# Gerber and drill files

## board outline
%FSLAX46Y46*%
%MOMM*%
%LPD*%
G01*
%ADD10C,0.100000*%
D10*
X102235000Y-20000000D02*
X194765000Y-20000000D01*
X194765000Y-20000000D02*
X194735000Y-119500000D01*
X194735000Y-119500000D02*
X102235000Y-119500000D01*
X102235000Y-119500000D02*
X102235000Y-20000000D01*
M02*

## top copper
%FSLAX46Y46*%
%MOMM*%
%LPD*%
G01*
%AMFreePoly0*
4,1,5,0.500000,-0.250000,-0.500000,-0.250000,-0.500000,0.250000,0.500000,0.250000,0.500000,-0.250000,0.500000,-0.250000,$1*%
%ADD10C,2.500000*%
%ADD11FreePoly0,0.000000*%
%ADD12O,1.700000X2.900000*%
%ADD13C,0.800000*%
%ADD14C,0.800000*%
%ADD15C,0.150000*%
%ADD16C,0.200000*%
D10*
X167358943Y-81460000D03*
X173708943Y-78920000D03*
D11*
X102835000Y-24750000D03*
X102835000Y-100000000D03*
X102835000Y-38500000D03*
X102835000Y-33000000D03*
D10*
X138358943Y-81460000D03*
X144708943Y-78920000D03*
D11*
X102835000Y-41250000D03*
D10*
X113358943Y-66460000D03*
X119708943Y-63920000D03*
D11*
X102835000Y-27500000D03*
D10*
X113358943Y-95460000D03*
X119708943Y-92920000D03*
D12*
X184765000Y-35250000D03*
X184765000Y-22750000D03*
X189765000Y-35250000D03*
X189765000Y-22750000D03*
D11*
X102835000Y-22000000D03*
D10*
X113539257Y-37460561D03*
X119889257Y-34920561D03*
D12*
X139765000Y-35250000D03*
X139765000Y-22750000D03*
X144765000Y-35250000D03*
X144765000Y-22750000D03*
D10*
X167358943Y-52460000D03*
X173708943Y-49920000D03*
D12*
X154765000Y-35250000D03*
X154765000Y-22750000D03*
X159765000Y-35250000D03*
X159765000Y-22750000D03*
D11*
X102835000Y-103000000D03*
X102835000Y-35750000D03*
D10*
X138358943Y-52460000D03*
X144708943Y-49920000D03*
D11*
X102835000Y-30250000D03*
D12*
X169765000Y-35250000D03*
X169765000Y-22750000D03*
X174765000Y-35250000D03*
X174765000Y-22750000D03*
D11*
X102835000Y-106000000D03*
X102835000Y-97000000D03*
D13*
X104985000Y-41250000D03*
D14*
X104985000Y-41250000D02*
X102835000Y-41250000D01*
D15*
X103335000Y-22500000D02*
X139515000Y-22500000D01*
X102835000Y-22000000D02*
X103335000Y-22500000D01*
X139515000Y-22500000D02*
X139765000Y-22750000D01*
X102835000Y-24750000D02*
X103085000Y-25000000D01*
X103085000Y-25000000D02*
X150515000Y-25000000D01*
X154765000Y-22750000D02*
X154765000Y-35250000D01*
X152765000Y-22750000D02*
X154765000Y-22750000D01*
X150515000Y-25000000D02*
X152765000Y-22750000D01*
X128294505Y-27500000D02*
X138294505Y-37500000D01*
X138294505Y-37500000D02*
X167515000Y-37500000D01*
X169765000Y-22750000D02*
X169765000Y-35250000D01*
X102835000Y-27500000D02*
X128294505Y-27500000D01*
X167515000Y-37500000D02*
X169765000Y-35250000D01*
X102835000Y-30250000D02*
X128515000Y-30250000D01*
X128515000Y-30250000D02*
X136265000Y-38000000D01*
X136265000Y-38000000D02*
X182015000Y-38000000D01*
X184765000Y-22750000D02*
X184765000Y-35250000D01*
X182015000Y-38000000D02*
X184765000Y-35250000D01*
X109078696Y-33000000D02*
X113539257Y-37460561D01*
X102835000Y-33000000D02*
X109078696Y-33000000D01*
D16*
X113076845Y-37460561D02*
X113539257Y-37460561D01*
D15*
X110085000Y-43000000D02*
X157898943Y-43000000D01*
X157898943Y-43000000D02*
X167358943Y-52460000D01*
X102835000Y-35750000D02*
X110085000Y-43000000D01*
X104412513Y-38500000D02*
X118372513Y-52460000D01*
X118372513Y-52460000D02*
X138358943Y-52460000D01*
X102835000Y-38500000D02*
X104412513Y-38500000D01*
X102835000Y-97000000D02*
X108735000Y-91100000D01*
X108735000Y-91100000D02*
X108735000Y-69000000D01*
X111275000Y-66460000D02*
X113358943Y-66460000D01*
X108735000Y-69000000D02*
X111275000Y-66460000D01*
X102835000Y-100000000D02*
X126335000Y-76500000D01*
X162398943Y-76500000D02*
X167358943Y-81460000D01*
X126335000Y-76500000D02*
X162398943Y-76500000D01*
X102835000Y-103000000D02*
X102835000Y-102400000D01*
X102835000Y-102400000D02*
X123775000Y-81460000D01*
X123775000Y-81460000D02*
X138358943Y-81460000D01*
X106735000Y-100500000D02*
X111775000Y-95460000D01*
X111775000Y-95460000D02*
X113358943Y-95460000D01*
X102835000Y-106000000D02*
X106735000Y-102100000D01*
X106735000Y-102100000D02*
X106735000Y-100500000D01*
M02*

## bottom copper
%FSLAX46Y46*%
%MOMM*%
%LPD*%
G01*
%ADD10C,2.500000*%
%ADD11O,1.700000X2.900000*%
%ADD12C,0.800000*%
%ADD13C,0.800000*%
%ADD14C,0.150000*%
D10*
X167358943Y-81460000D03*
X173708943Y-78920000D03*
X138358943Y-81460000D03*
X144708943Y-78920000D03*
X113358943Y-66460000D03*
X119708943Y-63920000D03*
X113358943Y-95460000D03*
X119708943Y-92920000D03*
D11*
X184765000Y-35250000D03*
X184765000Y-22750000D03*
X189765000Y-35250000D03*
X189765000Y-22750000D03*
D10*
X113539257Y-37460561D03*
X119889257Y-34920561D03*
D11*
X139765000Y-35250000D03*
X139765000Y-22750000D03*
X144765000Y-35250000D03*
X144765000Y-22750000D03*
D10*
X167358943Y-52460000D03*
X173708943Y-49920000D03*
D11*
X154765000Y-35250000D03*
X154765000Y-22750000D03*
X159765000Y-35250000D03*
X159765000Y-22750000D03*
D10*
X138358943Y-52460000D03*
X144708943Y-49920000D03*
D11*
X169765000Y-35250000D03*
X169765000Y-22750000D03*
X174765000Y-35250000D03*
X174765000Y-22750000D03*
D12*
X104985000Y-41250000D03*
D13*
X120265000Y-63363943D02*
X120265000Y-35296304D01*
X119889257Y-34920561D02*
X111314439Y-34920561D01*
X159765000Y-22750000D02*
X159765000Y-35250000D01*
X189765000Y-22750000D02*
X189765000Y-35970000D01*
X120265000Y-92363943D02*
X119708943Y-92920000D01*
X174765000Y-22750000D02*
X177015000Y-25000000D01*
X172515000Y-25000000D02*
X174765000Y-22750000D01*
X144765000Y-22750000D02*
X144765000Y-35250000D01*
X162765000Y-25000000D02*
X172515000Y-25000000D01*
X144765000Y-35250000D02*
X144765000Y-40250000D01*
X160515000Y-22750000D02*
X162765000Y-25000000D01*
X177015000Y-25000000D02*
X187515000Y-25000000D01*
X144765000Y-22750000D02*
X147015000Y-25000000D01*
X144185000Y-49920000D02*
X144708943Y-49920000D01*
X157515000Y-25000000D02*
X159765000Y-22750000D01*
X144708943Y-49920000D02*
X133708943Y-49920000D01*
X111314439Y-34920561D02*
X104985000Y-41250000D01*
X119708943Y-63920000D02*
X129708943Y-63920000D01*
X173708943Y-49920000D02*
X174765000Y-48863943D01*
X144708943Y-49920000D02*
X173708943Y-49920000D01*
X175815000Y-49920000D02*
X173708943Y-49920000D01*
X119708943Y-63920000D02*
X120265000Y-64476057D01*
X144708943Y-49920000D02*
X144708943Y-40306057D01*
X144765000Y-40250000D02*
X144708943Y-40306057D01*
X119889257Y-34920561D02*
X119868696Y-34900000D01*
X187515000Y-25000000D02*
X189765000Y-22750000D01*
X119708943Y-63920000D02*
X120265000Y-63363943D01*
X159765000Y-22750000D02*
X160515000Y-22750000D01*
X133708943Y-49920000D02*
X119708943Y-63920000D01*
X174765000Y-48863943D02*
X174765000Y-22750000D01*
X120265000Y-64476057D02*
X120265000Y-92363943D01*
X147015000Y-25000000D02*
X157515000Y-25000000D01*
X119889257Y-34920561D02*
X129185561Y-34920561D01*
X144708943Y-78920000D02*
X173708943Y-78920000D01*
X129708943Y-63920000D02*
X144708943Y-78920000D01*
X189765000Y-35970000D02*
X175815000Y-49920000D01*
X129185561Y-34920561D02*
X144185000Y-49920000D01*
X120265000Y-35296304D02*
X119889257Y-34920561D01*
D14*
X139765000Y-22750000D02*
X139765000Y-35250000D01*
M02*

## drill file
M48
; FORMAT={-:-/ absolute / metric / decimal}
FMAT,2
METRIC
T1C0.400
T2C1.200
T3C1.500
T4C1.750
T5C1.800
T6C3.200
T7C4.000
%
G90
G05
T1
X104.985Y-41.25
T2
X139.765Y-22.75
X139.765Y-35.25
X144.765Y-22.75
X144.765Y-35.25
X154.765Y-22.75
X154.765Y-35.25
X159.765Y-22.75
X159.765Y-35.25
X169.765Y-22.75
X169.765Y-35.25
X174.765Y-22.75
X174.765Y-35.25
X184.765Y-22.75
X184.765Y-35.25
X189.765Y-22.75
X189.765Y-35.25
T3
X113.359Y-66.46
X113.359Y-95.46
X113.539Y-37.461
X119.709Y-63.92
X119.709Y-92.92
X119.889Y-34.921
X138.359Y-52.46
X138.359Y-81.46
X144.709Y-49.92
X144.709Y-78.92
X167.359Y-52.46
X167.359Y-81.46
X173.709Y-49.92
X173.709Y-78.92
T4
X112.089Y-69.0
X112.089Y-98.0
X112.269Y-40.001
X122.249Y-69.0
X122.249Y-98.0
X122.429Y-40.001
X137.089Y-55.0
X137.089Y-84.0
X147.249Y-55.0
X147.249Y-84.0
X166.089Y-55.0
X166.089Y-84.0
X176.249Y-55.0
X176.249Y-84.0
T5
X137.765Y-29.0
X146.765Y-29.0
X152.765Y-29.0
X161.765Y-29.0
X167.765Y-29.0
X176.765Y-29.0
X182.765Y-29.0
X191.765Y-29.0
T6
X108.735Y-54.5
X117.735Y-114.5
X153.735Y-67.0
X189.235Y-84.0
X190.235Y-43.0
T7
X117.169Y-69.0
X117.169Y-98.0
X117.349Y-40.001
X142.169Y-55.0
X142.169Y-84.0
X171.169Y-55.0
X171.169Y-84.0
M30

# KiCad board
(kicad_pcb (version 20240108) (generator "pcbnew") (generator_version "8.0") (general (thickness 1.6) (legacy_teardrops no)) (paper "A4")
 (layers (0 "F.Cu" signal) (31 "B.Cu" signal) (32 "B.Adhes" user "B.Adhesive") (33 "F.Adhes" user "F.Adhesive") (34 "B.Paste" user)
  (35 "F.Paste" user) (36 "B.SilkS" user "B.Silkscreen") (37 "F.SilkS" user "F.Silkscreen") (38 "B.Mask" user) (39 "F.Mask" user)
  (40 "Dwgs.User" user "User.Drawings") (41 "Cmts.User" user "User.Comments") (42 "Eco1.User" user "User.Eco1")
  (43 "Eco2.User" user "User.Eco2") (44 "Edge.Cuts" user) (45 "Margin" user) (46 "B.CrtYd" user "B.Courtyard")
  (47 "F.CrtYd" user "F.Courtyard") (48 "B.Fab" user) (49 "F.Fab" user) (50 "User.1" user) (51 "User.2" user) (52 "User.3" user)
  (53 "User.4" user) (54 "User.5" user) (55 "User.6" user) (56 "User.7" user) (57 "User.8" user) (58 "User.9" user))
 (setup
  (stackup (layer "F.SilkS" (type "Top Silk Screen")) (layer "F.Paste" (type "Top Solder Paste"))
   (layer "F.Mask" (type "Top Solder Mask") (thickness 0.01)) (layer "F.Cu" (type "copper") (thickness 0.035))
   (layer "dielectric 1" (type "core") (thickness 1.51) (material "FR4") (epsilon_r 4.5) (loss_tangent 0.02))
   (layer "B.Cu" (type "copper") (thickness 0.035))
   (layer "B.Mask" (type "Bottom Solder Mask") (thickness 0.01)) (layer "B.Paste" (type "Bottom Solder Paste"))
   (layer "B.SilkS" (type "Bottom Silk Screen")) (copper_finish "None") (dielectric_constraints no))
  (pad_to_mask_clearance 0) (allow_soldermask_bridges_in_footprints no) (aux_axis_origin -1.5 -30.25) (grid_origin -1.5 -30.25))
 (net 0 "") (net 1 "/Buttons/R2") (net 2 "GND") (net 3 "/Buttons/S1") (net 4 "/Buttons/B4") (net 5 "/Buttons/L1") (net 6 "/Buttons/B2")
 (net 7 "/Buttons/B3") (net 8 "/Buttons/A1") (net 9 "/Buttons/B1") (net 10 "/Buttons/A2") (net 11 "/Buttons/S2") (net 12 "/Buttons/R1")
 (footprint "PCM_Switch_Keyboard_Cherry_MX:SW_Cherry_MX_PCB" (layer "F.Cu") (at 171.168943 84)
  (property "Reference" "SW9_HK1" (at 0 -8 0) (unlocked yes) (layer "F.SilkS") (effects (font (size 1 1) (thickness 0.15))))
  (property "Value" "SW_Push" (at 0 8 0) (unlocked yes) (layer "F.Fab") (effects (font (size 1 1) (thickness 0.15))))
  (pad "" np_thru_hole circle (at -5.08 0) (size 1.75 1.75) (drill 1.75) (layers "*.Cu" "*.Mask"))
  (pad "" np_thru_hole circle (at 0 0) (size 4 4) (drill 4) (layers "*.Cu" "*.Mask"))
  (pad "" np_thru_hole circle (at 5.08 0) (size 1.75 1.75) (drill 1.75) (layers "*.Cu" "*.Mask"))
  (pad "1" thru_hole circle (at -3.81 -2.54) (size 2.5 2.5) (drill 1.5) (layers "*.Cu" "*.Mask") (remove_unused_layers no)
   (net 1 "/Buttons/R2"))
  (pad "2" thru_hole circle (at 2.54 -5.08) (size 2.5 2.5) (drill 1.5) (layers "*.Cu" "*.Mask") (remove_unused_layers no) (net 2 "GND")))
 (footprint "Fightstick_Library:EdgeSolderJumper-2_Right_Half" (layer "F.Cu") (at 102.185 24.75)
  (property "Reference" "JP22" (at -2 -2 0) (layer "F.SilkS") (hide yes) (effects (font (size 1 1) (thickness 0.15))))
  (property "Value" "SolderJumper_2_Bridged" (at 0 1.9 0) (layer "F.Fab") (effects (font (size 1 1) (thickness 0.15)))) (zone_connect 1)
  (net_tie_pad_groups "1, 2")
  (pad "2" smd custom (at 0.65 0) (size 1 0.5) (layers "F.Cu" "F.Mask") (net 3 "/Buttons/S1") (zone_connect 2) (thermal_bridge_angle 45)
   (options (clearance outline) (anchor rect)) (primitives)))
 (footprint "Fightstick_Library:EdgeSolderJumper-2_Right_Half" (layer "F.Cu") (at 102.185 100)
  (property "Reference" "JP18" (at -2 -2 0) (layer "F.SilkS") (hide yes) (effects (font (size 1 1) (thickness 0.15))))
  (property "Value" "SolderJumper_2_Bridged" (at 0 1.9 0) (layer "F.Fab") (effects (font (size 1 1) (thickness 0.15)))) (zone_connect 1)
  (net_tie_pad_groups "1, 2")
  (pad "2" smd custom (at 0.65 0) (size 1 0.5) (layers "F.Cu" "F.Mask") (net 1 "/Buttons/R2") (zone_connect 2) (thermal_bridge_angle 45)
   (options (clearance outline) (anchor rect)) (primitives)))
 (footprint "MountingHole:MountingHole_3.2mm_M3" (layer "F.Cu") (at 117.735 114.5)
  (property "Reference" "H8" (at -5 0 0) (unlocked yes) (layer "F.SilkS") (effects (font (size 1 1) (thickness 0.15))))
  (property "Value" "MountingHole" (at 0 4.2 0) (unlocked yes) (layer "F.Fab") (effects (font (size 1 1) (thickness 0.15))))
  (pad "" np_thru_hole circle (at 0 0) (size 3.2 3.2) (drill 3.2) (layers "*.Cu" "*.Mask")))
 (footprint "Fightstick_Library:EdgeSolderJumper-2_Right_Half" (layer "F.Cu") (at 102.185 38.5)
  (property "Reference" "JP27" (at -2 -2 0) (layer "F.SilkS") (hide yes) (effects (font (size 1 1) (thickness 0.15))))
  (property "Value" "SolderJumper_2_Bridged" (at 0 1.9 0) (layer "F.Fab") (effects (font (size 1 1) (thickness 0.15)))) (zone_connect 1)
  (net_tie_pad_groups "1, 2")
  (pad "2" smd custom (at 0.65 0) (size 1 0.5) (layers "F.Cu" "F.Mask") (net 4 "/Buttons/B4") (zone_connect 2) (thermal_bridge_angle 45)
   (options (clearance outline) (anchor rect)) (primitives)))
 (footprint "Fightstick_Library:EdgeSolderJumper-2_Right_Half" (layer "F.Cu") (at 102.185 33)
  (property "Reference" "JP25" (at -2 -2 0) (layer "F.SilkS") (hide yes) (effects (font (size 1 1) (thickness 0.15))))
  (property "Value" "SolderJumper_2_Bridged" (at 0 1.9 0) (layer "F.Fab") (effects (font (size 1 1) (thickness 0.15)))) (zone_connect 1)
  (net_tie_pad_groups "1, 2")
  (pad "2" smd custom (at 0.65 0) (size 1 0.5) (layers "F.Cu" "F.Mask") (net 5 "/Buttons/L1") (zone_connect 2) (thermal_bridge_angle 45)
   (options (clearance outline) (anchor rect)) (primitives)))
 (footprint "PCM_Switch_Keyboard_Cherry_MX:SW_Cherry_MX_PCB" (layer "F.Cu") (at 142.168943 84)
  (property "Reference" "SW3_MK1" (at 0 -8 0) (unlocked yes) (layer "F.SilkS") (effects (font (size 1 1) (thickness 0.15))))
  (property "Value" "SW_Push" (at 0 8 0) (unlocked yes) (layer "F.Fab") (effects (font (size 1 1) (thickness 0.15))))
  (pad "" np_thru_hole circle (at -5.08 0) (size 1.75 1.75) (drill 1.75) (layers "*.Cu" "*.Mask"))
  (pad "" np_thru_hole circle (at 0 0) (size 4 4) (drill 4) (layers "*.Cu" "*.Mask"))
  (pad "" np_thru_hole circle (at 5.08 0) (size 1.75 1.75) (drill 1.75) (layers "*.Cu" "*.Mask"))
  (pad "1" thru_hole circle (at -3.81 -2.54) (size 2.5 2.5) (drill 1.5) (layers "*.Cu" "*.Mask") (remove_unused_layers no)
   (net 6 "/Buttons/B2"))
  (pad "2" thru_hole circle (at 2.54 -5.08) (size 2.5 2.5) (drill 1.5) (layers "*.Cu" "*.Mask") (remove_unused_layers no) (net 2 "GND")))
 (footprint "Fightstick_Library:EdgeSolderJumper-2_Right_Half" (layer "F.Cu") (at 102.185 41.25)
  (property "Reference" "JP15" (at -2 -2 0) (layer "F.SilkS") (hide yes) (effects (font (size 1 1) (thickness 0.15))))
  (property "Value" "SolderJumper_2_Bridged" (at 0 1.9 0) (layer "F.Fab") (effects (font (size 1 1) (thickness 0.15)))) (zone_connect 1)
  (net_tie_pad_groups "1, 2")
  (pad "2" smd custom (at 0.65 0) (size 1 0.5) (layers "F.Cu" "F.Mask") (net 2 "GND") (zone_connect 2) (thermal_bridge_angle 45)
   (options (clearance outline) (anchor rect)) (primitives)))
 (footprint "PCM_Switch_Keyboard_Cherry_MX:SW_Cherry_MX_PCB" (layer "F.Cu") (at 117.168943 69)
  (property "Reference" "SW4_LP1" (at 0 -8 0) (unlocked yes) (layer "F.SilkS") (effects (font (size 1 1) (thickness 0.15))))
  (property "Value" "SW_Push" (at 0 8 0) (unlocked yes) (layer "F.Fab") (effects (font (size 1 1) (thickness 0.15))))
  (pad "" np_thru_hole circle (at -5.08 0) (size 1.75 1.75) (drill 1.75) (layers "*.Cu" "*.Mask"))
  (pad "" np_thru_hole circle (at 0 0) (size 4 4) (drill 4) (layers "*.Cu" "*.Mask"))
  (pad "" np_thru_hole circle (at 5.08 0) (size 1.75 1.75) (drill 1.75) (layers "*.Cu" "*.Mask"))
  (pad "1" thru_hole circle (at -3.81 -2.54) (size 2.5 2.5) (drill 1.5) (layers "*.Cu" "*.Mask") (remove_unused_layers no)
   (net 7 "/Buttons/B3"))
  (pad "2" thru_hole circle (at 2.54 -5.08) (size 2.5 2.5) (drill 1.5) (layers "*.Cu" "*.Mask") (remove_unused_layers no) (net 2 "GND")))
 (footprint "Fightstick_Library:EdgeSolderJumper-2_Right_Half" (layer "F.Cu") (at 102.185 27.5)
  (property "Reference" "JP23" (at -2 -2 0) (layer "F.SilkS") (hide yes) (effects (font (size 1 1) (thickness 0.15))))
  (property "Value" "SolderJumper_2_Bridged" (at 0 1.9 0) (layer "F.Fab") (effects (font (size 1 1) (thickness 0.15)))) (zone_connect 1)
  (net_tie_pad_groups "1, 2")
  (pad "2" smd custom (at 0.65 0) (size 1 0.5) (layers "F.Cu" "F.Mask") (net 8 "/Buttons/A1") (zone_connect 2) (thermal_bridge_angle 45)
   (options (clearance outline) (anchor rect)) (primitives)))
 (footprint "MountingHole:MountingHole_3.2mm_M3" (layer "F.Cu") (at 190.235 43)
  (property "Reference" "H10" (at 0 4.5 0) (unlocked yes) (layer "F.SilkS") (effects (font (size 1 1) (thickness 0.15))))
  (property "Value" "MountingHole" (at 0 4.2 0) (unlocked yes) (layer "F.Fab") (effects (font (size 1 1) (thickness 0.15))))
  (pad "" np_thru_hole circle (at 0 0) (size 3.2 3.2) (drill 3.2) (layers "*.Cu" "*.Mask")))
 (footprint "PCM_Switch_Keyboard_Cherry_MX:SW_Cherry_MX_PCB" (layer "F.Cu") (at 117.168943 98)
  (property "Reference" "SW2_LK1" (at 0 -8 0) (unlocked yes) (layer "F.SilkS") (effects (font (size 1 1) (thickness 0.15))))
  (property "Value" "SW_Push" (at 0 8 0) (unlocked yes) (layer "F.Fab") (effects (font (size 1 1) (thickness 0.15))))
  (pad "" np_thru_hole circle (at -5.08 0) (size 1.75 1.75) (drill 1.75) (layers "*.Cu" "*.Mask"))
  (pad "" np_thru_hole circle (at 0 0) (size 4 4) (drill 4) (layers "*.Cu" "*.Mask"))
  (pad "" np_thru_hole circle (at 5.08 0) (size 1.75 1.75) (drill 1.75) (layers "*.Cu" "*.Mask"))
  (pad "1" thru_hole circle (at -3.81 -2.54) (size 2.5 2.5) (drill 1.5) (layers "*.Cu" "*.Mask") (remove_unused_layers no)
   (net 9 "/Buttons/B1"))
  (pad "2" thru_hole circle (at 2.54 -5.08) (size 2.5 2.5) (drill 1.5) (layers "*.Cu" "*.Mask") (remove_unused_layers no) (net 2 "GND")))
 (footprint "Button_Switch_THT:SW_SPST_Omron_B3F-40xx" (layer "F.Cu") (at 184.765 35.25 90)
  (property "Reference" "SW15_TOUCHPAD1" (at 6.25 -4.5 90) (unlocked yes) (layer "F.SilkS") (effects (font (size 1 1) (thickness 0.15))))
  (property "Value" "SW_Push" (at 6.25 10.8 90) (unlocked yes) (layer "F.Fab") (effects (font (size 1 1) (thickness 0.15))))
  (pad "" np_thru_hole circle (at 6.25 -2 90) (size 1.8 1.8) (drill 1.8) (layers "F&B.Cu" "*.Mask"))
  (pad "" np_thru_hole circle (at 6.25 7 90) (size 1.8 1.8) (drill 1.8) (layers "F&B.Cu" "*.Mask"))
  (pad "1" thru_hole oval (at 0 0 90) (size 2.9 1.7) (drill 1.2) (layers "*.Cu" "*.Mask") (remove_unused_layers no) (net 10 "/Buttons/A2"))
  (pad "1" thru_hole oval (at 12.5 0 90) (size 2.9 1.7) (drill 1.2) (layers "*.Cu" "*.Mask") (remove_unused_layers no)
   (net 10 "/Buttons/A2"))
  (pad "2" thru_hole oval (at 0 5 90) (size 2.9 1.7) (drill 1.2) (layers "*.Cu" "*.Mask") (remove_unused_layers no) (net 2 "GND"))
  (pad "2" thru_hole oval (at 12.5 5 90) (size 2.9 1.7) (drill 1.2) (layers "*.Cu" "*.Mask") (remove_unused_layers no) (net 2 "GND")))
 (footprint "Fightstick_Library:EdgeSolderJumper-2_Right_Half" (layer "F.Cu") (at 102.185 22)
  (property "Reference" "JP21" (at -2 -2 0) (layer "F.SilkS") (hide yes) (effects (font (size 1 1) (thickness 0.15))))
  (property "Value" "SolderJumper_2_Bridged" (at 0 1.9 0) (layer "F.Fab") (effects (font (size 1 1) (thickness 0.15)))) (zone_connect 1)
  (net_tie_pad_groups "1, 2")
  (pad "2" smd custom (at 0.65 0) (size 1 0.5) (layers "F.Cu" "F.Mask") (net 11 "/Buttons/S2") (zone_connect 2) (thermal_bridge_angle 45)
   (options (clearance outline) (anchor rect)) (primitives)))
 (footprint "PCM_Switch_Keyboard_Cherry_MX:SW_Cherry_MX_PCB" (layer "F.Cu") (at 117.349257 40.000561)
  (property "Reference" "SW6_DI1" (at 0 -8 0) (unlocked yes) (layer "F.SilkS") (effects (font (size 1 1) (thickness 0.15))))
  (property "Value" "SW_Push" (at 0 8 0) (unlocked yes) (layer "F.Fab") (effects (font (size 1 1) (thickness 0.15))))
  (pad "" np_thru_hole circle (at -5.08 0) (size 1.75 1.75) (drill 1.75) (layers "*.Cu" "*.Mask"))
  (pad "" np_thru_hole circle (at 0 0) (size 4 4) (drill 4) (layers "*.Cu" "*.Mask"))
  (pad "" np_thru_hole circle (at 5.08 0) (size 1.75 1.75) (drill 1.75) (layers "*.Cu" "*.Mask"))
  (pad "1" thru_hole circle (at -3.81 -2.54) (size 2.5 2.5) (drill 1.5) (layers "*.Cu" "*.Mask") (remove_unused_layers no)
   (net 5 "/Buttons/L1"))
  (pad "2" thru_hole circle (at 2.54 -5.08) (size 2.5 2.5) (drill 1.5) (layers "*.Cu" "*.Mask") (remove_unused_layers no) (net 2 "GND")))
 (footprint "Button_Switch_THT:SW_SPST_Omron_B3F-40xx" (layer "F.Cu") (at 139.765 35.25 90)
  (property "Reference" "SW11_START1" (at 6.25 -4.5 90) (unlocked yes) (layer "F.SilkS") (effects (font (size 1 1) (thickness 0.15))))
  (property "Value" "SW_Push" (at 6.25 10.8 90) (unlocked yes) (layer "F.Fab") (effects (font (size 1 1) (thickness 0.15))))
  (pad "" np_thru_hole circle (at 6.25 -2 90) (size 1.8 1.8) (drill 1.8) (layers "F&B.Cu" "*.Mask"))
  (pad "" np_thru_hole circle (at 6.25 7 90) (size 1.8 1.8) (drill 1.8) (layers "F&B.Cu" "*.Mask"))
  (pad "1" thru_hole oval (at 0 0 90) (size 2.9 1.7) (drill 1.2) (layers "*.Cu" "*.Mask") (remove_unused_layers no) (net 11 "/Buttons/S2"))
  (pad "1" thru_hole oval (at 12.5 0 90) (size 2.9 1.7) (drill 1.2) (layers "*.Cu" "*.Mask") (remove_unused_layers no)
   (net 11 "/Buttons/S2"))
  (pad "2" thru_hole oval (at 0 5 90) (size 2.9 1.7) (drill 1.2) (layers "*.Cu" "*.Mask") (remove_unused_layers no) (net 2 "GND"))
  (pad "2" thru_hole oval (at 12.5 5 90) (size 2.9 1.7) (drill 1.2) (layers "*.Cu" "*.Mask") (remove_unused_layers no) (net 2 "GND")))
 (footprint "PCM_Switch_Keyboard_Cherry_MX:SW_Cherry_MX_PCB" (layer "F.Cu") (at 171.168943 55)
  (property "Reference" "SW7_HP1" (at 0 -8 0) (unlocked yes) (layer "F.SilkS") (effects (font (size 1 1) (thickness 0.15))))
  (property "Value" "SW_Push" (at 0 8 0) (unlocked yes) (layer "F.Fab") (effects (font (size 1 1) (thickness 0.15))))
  (pad "" np_thru_hole circle (at -5.08 0) (size 1.75 1.75) (drill 1.75) (layers "*.Cu" "*.Mask"))
  (pad "" np_thru_hole circle (at 0 0) (size 4 4) (drill 4) (layers "*.Cu" "*.Mask"))
  (pad "" np_thru_hole circle (at 5.08 0) (size 1.75 1.75) (drill 1.75) (layers "*.Cu" "*.Mask"))
  (pad "1" thru_hole circle (at -3.81 -2.54) (size 2.5 2.5) (drill 1.5) (layers "*.Cu" "*.Mask") (remove_unused_layers no)
   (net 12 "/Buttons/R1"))
  (pad "2" thru_hole circle (at 2.54 -5.08) (size 2.5 2.5) (drill 1.5) (layers "*.Cu" "*.Mask") (remove_unused_layers no) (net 2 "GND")))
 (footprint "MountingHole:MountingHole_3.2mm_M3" (layer "F.Cu") (at 153.735 67)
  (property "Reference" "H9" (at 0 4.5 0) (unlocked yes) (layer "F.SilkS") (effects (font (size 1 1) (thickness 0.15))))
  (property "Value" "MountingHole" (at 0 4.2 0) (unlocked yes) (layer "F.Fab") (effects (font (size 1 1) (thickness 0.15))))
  (pad "" np_thru_hole circle (at 0 0) (size 3.2 3.2) (drill 3.2) (layers "*.Cu" "*.Mask")))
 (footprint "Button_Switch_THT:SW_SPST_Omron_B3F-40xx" (layer "F.Cu") (at 154.765 35.25 90)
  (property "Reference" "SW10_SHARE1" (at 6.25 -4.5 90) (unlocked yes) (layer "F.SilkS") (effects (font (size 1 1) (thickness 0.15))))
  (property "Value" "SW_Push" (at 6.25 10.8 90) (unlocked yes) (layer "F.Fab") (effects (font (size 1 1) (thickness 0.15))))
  (pad "" np_thru_hole circle (at 6.25 -2 90) (size 1.8 1.8) (drill 1.8) (layers "F&B.Cu" "*.Mask"))
  (pad "" np_thru_hole circle (at 6.25 7 90) (size 1.8 1.8) (drill 1.8) (layers "F&B.Cu" "*.Mask"))
  (pad "1" thru_hole oval (at 0 0 90) (size 2.9 1.7) (drill 1.2) (layers "*.Cu" "*.Mask") (remove_unused_layers no) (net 3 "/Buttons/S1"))
  (pad "1" thru_hole oval (at 12.5 0 90) (size 2.9 1.7) (drill 1.2) (layers "*.Cu" "*.Mask") (remove_unused_layers no) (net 3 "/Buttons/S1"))
  (pad "2" thru_hole oval (at 0 5 90) (size 2.9 1.7) (drill 1.2) (layers "*.Cu" "*.Mask") (remove_unused_layers no) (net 2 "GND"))
  (pad "2" thru_hole oval (at 12.5 5 90) (size 2.9 1.7) (drill 1.2) (layers "*.Cu" "*.Mask") (remove_unused_layers no) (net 2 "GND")))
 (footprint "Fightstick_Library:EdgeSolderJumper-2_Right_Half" (layer "F.Cu") (at 102.185 103)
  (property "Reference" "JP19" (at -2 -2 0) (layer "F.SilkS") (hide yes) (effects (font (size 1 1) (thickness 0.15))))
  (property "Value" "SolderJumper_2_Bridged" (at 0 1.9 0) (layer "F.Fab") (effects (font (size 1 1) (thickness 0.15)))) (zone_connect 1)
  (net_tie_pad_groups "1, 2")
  (pad "2" smd custom (at 0.65 0) (size 1 0.5) (layers "F.Cu" "F.Mask") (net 6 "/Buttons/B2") (zone_connect 2) (thermal_bridge_angle 45)
   (options (clearance outline) (anchor rect)) (primitives)))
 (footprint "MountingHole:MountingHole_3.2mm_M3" (layer "F.Cu") (at 108.735 54.5)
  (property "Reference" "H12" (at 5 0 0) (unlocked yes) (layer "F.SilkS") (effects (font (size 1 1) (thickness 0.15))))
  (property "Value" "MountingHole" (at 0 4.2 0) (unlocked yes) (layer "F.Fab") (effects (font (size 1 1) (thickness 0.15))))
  (pad "" np_thru_hole circle (at 0 0) (size 3.2 3.2) (drill 3.2) (layers "*.Cu" "*.Mask")))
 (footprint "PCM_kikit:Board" (layer "F.Cu") (at 112.235 20)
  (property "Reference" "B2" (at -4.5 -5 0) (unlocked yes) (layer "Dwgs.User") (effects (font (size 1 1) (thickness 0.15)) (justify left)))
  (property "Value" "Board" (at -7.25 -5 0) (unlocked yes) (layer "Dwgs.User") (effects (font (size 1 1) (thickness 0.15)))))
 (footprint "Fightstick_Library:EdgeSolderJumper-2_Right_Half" (layer "F.Cu") (at 102.185 35.75)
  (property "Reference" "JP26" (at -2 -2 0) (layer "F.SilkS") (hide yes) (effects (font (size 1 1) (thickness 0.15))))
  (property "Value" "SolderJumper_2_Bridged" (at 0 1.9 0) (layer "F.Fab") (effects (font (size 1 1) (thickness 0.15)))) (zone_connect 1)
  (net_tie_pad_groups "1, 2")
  (pad "2" smd custom (at 0.65 0) (size 1 0.5) (layers "F.Cu" "F.Mask") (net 12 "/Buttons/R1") (zone_connect 2) (thermal_bridge_angle 45)
   (options (clearance outline) (anchor rect)) (primitives)))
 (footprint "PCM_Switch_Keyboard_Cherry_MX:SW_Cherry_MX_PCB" (layer "F.Cu") (at 142.168943 55)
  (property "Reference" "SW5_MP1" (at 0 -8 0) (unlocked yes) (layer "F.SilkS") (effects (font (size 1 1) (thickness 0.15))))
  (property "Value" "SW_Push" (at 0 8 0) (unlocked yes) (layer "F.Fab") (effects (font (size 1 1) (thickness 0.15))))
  (pad "" np_thru_hole circle (at -5.08 0) (size 1.75 1.75) (drill 1.75) (layers "*.Cu" "*.Mask"))
  (pad "" np_thru_hole circle (at 0 0) (size 4 4) (drill 4) (layers "*.Cu" "*.Mask"))
  (pad "" np_thru_hole circle (at 5.08 0) (size 1.75 1.75) (drill 1.75) (layers "*.Cu" "*.Mask"))
  (pad "1" thru_hole circle (at -3.81 -2.54) (size 2.5 2.5) (drill 1.5) (layers "*.Cu" "*.Mask") (remove_unused_layers no)
   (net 4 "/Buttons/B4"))
  (pad "2" thru_hole circle (at 2.54 -5.08) (size 2.5 2.5) (drill 1.5) (layers "*.Cu" "*.Mask") (remove_unused_layers no) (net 2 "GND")))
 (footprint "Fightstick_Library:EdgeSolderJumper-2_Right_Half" (layer "F.Cu") (at 102.185 30.25)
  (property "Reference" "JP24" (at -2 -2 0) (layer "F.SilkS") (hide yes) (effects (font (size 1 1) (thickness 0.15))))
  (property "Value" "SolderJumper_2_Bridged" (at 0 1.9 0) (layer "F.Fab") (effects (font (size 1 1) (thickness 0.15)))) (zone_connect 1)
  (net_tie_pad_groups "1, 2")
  (pad "2" smd custom (at 0.65 0) (size 1 0.5) (layers "F.Cu" "F.Mask") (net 10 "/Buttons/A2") (zone_connect 2) (thermal_bridge_angle 45)
   (options (clearance outline) (anchor rect)) (primitives)))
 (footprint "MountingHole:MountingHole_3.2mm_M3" (layer "F.Cu") (at 189.235 84)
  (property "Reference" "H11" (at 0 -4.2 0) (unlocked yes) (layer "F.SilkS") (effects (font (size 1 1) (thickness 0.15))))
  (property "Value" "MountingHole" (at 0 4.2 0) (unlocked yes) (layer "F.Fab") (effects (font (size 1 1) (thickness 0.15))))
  (pad "" np_thru_hole circle (at 0 0) (size 3.2 3.2) (drill 3.2) (layers "*.Cu" "*.Mask")))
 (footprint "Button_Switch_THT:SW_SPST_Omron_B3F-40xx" (layer "F.Cu") (at 169.765 35.25 90)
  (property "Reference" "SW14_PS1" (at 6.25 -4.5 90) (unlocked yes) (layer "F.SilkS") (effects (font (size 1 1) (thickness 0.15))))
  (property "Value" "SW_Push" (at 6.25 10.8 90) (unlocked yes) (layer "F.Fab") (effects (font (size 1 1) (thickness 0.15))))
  (pad "" np_thru_hole circle (at 6.25 -2 90) (size 1.8 1.8) (drill 1.8) (layers "F&B.Cu" "*.Mask"))
  (pad "" np_thru_hole circle (at 6.25 7 90) (size 1.8 1.8) (drill 1.8) (layers "F&B.Cu" "*.Mask"))
  (pad "1" thru_hole oval (at 0 0 90) (size 2.9 1.7) (drill 1.2) (layers "*.Cu" "*.Mask") (remove_unused_layers no) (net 8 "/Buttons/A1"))
  (pad "1" thru_hole oval (at 12.5 0 90) (size 2.9 1.7) (drill 1.2) (layers "*.Cu" "*.Mask") (remove_unused_layers no) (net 8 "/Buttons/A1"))
  (pad "2" thru_hole oval (at 0 5 90) (size 2.9 1.7) (drill 1.2) (layers "*.Cu" "*.Mask") (remove_unused_layers no) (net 2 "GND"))
  (pad "2" thru_hole oval (at 12.5 5 90) (size 2.9 1.7) (drill 1.2) (layers "*.Cu" "*.Mask") (remove_unused_layers no) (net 2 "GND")))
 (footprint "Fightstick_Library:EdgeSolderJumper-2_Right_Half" (layer "F.Cu") (at 102.185 106)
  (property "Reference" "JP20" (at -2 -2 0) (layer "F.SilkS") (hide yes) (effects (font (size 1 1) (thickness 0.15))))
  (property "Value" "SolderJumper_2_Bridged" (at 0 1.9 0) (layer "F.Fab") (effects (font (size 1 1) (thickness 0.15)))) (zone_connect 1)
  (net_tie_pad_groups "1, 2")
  (pad "2" smd custom (at 0.65 0) (size 1 0.5) (layers "F.Cu" "F.Mask") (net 9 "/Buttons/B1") (zone_connect 2) (thermal_bridge_angle 45)
   (options (clearance outline) (anchor rect)) (primitives)))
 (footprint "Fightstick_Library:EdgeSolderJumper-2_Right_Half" (layer "F.Cu") (at 102.185 97)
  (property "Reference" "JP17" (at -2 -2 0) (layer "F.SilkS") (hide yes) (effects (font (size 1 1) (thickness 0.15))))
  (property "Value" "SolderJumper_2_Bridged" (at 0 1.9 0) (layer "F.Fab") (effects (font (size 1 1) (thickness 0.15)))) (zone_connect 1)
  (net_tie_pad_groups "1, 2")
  (pad "2" smd custom (at 0.65 0) (size 1 0.5) (layers "F.Cu" "F.Mask") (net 7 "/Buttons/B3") (zone_connect 2) (thermal_bridge_angle 45)
   (options (clearance outline) (anchor rect)) (primitives)))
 (gr_line (start 102.235 20) (end 194.765 20) (stroke (width 0.1) (type default)) (layer "Edge.Cuts"))
 (gr_line (start 194.765 20) (end 194.735 119.5) (stroke (width 0.1) (type default)) (layer "Edge.Cuts"))
 (gr_line (start 194.735 119.5) (end 102.235 119.5) (stroke (width 0.1) (type default)) (layer "Edge.Cuts"))
 (gr_line (start 102.235 119.5) (end 102.235 20) (stroke (width 0.1) (type default)) (layer "Edge.Cuts"))
 (segment (start 104.985 41.25) (end 102.835 41.25) (width 0.8) (layer "F.Cu") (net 2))
 (via (at 104.985 41.25) (size 0.8) (drill 0.4) (layers "F.Cu" "B.Cu") (free yes) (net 2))
 (segment (start 120.265 63.363943) (end 120.265 35.296304) (width 0.8) (layer "B.Cu") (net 2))
 (segment (start 119.889257 34.920561) (end 111.314439 34.920561) (width 0.8) (layer "B.Cu") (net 2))
 (segment (start 159.765 22.75) (end 159.765 35.25) (width 0.8) (layer "B.Cu") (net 2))
 (segment (start 189.765 22.75) (end 189.765 35.97) (width 0.8) (layer "B.Cu") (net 2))
 (segment (start 120.265 92.363943) (end 119.708943 92.92) (width 0.8) (layer "B.Cu") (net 2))
 (segment (start 174.765 22.75) (end 177.015 25) (width 0.8) (layer "B.Cu") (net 2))
 (segment (start 172.515 25) (end 174.765 22.75) (width 0.8) (layer "B.Cu") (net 2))
 (segment (start 144.765 22.75) (end 144.765 35.25) (width 0.8) (layer "B.Cu") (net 2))
 (segment (start 162.765 25) (end 172.515 25) (width 0.8) (layer "B.Cu") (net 2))
 (segment (start 144.765 35.25) (end 144.765 40.25) (width 0.8) (layer "B.Cu") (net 2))
 (segment (start 160.515 22.75) (end 162.765 25) (width 0.8) (layer "B.Cu") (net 2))
 (segment (start 177.015 25) (end 187.515 25) (width 0.8) (layer "B.Cu") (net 2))
 (segment (start 144.765 22.75) (end 147.015 25) (width 0.8) (layer "B.Cu") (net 2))
 (segment (start 144.185 49.92) (end 144.708943 49.92) (width 0.8) (layer "B.Cu") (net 2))
 (segment (start 157.515 25) (end 159.765 22.75) (width 0.8) (layer "B.Cu") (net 2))
 (segment (start 144.708943 49.92) (end 133.708943 49.92) (width 0.8) (layer "B.Cu") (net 2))
 (segment (start 111.314439 34.920561) (end 104.985 41.25) (width 0.8) (layer "B.Cu") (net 2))
 (segment (start 119.708943 63.92) (end 129.708943 63.92) (width 0.8) (layer "B.Cu") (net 2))
 (segment (start 173.708943 49.92) (end 174.765 48.863943) (width 0.8) (layer "B.Cu") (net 2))
 (segment (start 144.708943 49.92) (end 173.708943 49.92) (width 0.8) (layer "B.Cu") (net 2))
 (segment (start 175.815 49.92) (end 173.708943 49.92) (width 0.8) (layer "B.Cu") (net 2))
 (segment (start 119.708943 63.92) (end 120.265 64.476057) (width 0.8) (layer "B.Cu") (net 2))
 (segment (start 144.708943 49.92) (end 144.708943 40.306057) (width 0.8) (layer "B.Cu") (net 2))
 (segment (start 144.765 40.25) (end 144.708943 40.306057) (width 0.8) (layer "B.Cu") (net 2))
 (segment (start 119.889257 34.920561) (end 119.868696 34.9) (width 0.8) (layer "B.Cu") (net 2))
 (segment (start 187.515 25) (end 189.765 22.75) (width 0.8) (layer "B.Cu") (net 2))
 (segment (start 119.708943 63.92) (end 120.265 63.363943) (width 0.8) (layer "B.Cu") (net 2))
 (segment (start 159.765 22.75) (end 160.515 22.75) (width 0.8) (layer "B.Cu") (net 2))
 (segment (start 133.708943 49.92) (end 119.708943 63.92) (width 0.8) (layer "B.Cu") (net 2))
 (segment (start 174.765 48.863943) (end 174.765 22.75) (width 0.8) (layer "B.Cu") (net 2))
 (segment (start 120.265 64.476057) (end 120.265 92.363943) (width 0.8) (layer "B.Cu") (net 2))
 (segment (start 147.015 25) (end 157.515 25) (width 0.8) (layer "B.Cu") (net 2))
 (segment (start 119.889257 34.920561) (end 129.185561 34.920561) (width 0.8) (layer "B.Cu") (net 2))
 (segment (start 144.708943 78.92) (end 173.708943 78.92) (width 0.8) (layer "B.Cu") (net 2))
 (segment (start 129.708943 63.92) (end 144.708943 78.92) (width 0.8) (layer "B.Cu") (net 2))
 (segment (start 189.765 35.97) (end 175.815 49.92) (width 0.8) (layer "B.Cu") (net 2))
 (segment (start 129.185561 34.920561) (end 144.185 49.92) (width 0.8) (layer "B.Cu") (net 2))
 (segment (start 120.265 35.296304) (end 119.889257 34.920561) (width 0.8) (layer "B.Cu") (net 2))
 (segment (start 103.335 22.5) (end 139.515 22.5) (width 0.15) (layer "F.Cu") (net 11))
 (segment (start 102.835 22) (end 103.335 22.5) (width 0.15) (layer "F.Cu") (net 11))
 (segment (start 139.515 22.5) (end 139.765 22.75) (width 0.15) (layer "F.Cu") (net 11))
 (segment (start 139.765 22.75) (end 139.765 35.25) (width 0.15) (layer "B.Cu") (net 11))
 (segment (start 102.835 24.75) (end 103.085 25) (width 0.15) (layer "F.Cu") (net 3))
 (segment (start 103.085 25) (end 150.515 25) (width 0.15) (layer "F.Cu") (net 3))
 (segment (start 154.765 22.75) (end 154.765 35.25) (width 0.15) (layer "F.Cu") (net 3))
 (segment (start 152.765 22.75) (end 154.765 22.75) (width 0.15) (layer "F.Cu") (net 3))
 (segment (start 150.515 25) (end 152.765 22.75) (width 0.15) (layer "F.Cu") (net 3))
 (segment (start 128.294505 27.5) (end 138.294505 37.5) (width 0.15) (layer "F.Cu") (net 8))
 (segment (start 138.294505 37.5) (end 167.515 37.5) (width 0.15) (layer "F.Cu") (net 8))
 (segment (start 169.765 22.75) (end 169.765 35.25) (width 0.15) (layer "F.Cu") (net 8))
 (segment (start 102.835 27.5) (end 128.294505 27.5) (width 0.15) (layer "F.Cu") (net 8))
 (segment (start 167.515 37.5) (end 169.765 35.25) (width 0.15) (layer "F.Cu") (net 8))
 (segment (start 102.835 30.25) (end 128.515 30.25) (width 0.15) (layer "F.Cu") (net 10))
 (segment (start 128.515 30.25) (end 136.265 38) (width 0.15) (layer "F.Cu") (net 10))
 (segment (start 136.265 38) (end 182.015 38) (width 0.15) (layer "F.Cu") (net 10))
 (segment (start 184.765 22.75) (end 184.765 35.25) (width 0.15) (layer "F.Cu") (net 10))
 (segment (start 182.015 38) (end 184.765 35.25) (width 0.15) (layer "F.Cu") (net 10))
 (segment (start 109.078696 33) (end 113.539257 37.460561) (width 0.15) (layer "F.Cu") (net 5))
 (segment (start 102.835 33) (end 109.078696 33) (width 0.15) (layer "F.Cu") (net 5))
 (segment (start 113.076845 37.460561) (end 113.539257 37.460561) (width 0.2) (layer "F.Cu") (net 5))
 (segment (start 110.085 43) (end 157.898943 43) (width 0.15) (layer "F.Cu") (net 12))
 (segment (start 157.898943 43) (end 167.358943 52.46) (width 0.15) (layer "F.Cu") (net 12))
 (segment (start 102.835 35.75) (end 110.085 43) (width 0.15) (layer "F.Cu") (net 12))
 (segment (start 104.412513 38.5) (end 118.372513 52.46) (width 0.15) (layer "F.Cu") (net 4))
 (segment (start 118.372513 52.46) (end 138.358943 52.46) (width 0.15) (layer "F.Cu") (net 4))
 (segment (start 102.835 38.5) (end 104.412513 38.5) (width 0.15) (layer "F.Cu") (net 4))
 (segment (start 102.835 97) (end 108.735 91.1) (width 0.15) (layer "F.Cu") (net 7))
 (segment (start 108.735 91.1) (end 108.735 69) (width 0.15) (layer "F.Cu") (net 7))
 (segment (start 111.275 66.46) (end 113.358943 66.46) (width 0.15) (layer "F.Cu") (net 7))
 (segment (start 108.735 69) (end 111.275 66.46) (width 0.15) (layer "F.Cu") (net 7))
 (segment (start 102.835 100) (end 126.335 76.5) (width 0.15) (layer "F.Cu") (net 1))
 (segment (start 162.398943 76.5) (end 167.358943 81.46) (width 0.15) (layer "F.Cu") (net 1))
 (segment (start 126.335 76.5) (end 162.398943 76.5) (width 0.15) (layer "F.Cu") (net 1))
 (segment (start 102.835 103) (end 102.835 102.4) (width 0.15) (layer "F.Cu") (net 6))
 (segment (start 102.835 102.4) (end 123.775 81.46) (width 0.15) (layer "F.Cu") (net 6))
 (segment (start 123.775 81.46) (end 138.358943 81.46) (width 0.15) (layer "F.Cu") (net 6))
 (segment (start 106.735 100.5) (end 111.775 95.46) (width 0.15) (layer "F.Cu") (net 9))
 (segment (start 111.775 95.46) (end 113.358943 95.46) (width 0.15) (layer "F.Cu") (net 9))
 (segment (start 102.835 106) (end 106.735 102.1) (width 0.15) (layer "F.Cu") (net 9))
 (segment (start 106.735 102.1) (end 106.735 100.5) (width 0.15) (layer "F.Cu") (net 9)))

